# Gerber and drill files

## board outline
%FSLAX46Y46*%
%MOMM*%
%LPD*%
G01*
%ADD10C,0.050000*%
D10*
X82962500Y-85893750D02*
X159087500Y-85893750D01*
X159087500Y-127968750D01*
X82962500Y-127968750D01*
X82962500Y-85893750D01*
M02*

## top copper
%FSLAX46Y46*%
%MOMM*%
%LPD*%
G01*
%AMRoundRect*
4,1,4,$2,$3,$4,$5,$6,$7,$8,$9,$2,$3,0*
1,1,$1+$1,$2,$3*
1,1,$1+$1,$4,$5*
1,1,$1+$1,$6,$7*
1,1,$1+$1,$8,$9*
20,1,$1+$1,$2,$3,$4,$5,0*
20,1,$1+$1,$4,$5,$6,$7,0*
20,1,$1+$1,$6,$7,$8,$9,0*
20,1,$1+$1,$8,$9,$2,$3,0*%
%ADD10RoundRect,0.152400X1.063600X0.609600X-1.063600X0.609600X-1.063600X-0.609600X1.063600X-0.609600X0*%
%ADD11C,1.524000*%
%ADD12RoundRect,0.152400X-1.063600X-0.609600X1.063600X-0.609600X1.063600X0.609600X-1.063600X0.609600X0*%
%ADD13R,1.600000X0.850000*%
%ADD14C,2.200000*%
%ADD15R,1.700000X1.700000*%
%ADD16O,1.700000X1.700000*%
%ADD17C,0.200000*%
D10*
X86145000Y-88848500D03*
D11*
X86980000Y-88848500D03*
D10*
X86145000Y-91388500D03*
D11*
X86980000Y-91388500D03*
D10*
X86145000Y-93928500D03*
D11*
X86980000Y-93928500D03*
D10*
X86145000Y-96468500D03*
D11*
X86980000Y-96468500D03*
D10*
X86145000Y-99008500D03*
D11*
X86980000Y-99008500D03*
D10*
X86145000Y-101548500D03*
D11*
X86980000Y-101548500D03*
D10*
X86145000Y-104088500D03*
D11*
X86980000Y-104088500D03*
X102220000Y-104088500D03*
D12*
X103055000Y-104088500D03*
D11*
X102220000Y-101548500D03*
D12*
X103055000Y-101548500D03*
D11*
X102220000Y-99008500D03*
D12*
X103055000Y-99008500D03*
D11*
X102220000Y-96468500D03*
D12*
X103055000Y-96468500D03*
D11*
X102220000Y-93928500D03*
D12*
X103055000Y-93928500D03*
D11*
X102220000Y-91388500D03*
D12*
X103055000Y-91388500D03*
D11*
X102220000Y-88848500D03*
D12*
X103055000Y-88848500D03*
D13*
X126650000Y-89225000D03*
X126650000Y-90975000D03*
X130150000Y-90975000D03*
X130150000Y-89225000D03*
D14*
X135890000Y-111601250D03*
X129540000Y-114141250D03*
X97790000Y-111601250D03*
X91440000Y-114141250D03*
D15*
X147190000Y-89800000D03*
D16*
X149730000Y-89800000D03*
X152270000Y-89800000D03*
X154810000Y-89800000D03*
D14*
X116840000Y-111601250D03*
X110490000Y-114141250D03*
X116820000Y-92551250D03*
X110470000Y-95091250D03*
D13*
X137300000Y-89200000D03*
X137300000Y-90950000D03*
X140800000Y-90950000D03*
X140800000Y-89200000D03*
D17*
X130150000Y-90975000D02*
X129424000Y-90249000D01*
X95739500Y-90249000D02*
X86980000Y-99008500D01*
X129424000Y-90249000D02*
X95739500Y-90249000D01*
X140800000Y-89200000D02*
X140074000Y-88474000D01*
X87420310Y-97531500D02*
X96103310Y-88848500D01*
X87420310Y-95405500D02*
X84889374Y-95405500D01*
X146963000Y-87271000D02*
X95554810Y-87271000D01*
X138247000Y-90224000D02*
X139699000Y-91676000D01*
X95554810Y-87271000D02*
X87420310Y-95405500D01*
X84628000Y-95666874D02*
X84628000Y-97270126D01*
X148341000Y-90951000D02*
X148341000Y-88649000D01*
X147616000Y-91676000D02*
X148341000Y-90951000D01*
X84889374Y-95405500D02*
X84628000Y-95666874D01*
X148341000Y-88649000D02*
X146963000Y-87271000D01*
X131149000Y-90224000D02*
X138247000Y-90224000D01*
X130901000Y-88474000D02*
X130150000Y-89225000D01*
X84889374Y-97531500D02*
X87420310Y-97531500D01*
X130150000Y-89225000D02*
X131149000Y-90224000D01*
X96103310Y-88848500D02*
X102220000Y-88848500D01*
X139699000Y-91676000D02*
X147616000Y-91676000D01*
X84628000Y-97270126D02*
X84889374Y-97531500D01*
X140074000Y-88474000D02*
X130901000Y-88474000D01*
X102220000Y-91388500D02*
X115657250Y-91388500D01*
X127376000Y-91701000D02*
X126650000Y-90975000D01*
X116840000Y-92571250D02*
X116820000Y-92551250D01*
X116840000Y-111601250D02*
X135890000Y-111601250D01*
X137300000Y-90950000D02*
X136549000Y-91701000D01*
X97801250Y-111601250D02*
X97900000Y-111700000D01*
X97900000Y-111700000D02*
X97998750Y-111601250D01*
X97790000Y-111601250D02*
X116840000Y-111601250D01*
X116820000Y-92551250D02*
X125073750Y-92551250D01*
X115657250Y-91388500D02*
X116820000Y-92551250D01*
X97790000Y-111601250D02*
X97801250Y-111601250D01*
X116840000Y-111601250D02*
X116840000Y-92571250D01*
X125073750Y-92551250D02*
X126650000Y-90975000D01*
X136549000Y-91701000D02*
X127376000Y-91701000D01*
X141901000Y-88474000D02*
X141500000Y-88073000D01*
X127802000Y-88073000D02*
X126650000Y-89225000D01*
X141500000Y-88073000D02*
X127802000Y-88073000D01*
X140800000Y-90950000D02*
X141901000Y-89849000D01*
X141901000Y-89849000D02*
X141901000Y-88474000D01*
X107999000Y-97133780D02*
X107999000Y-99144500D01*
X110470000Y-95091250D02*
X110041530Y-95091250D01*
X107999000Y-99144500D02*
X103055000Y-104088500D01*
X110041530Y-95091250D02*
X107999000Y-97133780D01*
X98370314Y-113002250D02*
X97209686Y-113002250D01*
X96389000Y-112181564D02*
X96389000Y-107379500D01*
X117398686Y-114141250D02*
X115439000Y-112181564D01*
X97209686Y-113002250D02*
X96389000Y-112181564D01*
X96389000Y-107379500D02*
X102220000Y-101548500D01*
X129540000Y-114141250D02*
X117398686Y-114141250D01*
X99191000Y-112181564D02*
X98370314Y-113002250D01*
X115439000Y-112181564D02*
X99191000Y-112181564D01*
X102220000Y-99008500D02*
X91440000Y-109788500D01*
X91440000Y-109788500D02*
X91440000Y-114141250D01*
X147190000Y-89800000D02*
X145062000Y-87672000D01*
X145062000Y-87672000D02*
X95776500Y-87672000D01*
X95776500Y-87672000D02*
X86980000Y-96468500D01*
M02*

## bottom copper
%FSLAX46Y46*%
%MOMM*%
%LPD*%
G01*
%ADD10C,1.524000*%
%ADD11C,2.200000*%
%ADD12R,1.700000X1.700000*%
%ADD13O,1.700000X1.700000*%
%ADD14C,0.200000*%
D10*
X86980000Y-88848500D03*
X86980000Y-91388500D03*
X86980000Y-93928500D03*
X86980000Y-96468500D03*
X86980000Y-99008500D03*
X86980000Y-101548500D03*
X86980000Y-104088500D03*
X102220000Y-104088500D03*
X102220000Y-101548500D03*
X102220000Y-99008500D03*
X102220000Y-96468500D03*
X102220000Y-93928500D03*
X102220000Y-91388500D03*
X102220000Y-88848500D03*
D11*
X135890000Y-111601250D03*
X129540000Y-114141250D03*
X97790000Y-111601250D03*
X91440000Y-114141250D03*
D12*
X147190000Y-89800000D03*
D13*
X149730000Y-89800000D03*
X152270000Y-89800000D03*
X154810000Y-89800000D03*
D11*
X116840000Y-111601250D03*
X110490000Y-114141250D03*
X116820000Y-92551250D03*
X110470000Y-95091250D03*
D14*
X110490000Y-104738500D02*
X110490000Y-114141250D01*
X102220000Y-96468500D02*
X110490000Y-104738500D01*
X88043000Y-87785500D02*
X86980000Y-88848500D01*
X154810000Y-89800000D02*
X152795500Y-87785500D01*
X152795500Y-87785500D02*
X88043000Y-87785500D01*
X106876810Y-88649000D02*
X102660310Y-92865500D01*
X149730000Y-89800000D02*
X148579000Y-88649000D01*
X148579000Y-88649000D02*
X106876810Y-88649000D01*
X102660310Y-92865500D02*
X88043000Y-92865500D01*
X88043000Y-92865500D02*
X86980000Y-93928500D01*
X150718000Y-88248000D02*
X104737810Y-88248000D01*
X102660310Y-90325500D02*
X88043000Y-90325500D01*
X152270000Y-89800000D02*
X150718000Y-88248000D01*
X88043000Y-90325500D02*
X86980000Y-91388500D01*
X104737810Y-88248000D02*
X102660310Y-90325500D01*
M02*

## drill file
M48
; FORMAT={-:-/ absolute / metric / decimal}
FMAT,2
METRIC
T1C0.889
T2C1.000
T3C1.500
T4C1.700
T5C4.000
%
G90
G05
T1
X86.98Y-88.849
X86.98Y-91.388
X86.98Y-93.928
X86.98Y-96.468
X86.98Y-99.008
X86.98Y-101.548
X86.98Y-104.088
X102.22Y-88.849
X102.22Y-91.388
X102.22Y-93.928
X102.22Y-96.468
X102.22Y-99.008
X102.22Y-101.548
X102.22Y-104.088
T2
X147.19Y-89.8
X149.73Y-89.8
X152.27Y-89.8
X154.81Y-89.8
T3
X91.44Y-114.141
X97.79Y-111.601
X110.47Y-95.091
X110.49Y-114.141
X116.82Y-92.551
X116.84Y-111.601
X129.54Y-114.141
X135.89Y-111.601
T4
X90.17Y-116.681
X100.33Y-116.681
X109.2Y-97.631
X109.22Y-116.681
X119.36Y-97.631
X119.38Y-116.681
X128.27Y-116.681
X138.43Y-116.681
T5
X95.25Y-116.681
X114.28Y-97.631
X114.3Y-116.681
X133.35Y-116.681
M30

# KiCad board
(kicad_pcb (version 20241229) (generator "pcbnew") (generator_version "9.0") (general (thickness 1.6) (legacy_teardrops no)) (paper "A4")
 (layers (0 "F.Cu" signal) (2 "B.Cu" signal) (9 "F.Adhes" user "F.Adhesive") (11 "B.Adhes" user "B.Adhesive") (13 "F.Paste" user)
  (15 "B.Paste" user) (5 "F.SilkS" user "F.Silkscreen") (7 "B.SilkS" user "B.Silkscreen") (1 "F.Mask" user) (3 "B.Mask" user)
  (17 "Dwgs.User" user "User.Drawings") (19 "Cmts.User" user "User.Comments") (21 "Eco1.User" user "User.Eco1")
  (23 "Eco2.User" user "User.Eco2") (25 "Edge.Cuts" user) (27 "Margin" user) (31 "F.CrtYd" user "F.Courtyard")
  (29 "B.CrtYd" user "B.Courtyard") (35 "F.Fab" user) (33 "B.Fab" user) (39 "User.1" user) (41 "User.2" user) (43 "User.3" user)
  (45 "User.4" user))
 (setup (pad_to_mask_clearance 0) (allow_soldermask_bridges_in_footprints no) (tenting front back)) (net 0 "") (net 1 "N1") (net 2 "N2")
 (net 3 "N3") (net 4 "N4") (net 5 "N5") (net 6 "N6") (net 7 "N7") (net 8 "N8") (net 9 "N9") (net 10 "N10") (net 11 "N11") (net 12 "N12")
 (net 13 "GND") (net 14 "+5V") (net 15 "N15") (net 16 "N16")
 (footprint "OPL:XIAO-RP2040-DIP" (layer "F.Cu") (at 94.6 96.4685)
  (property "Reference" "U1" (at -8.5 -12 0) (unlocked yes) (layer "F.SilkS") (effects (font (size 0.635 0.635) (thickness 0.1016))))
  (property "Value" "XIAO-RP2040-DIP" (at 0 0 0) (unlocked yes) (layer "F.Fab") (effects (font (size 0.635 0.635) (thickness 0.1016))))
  (pad "1" smd roundrect (at -8.455 -7.62 180) (size 2.432 1.524) (layers "F.Cu" "F.Mask") (roundrect_rratio 0.1) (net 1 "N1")
   (thermal_bridge_angle 45))
  (pad "1" thru_hole circle (at -7.62 -7.62 180) (size 1.524 1.524) (drill 0.889) (layers "*.Cu" "*.Mask") (remove_unused_layers no)
   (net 1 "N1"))
  (pad "2" smd roundrect (at -8.455 -5.08 180) (size 2.432 1.524) (layers "F.Cu" "F.Mask") (roundrect_rratio 0.1) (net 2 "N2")
   (thermal_bridge_angle 45))
  (pad "2" thru_hole circle (at -7.62 -5.08 180) (size 1.524 1.524) (drill 0.889) (layers "*.Cu" "*.Mask") (remove_unused_layers no)
   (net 2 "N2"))
  (pad "3" smd roundrect (at -8.455 -2.54 180) (size 2.432 1.524) (layers "F.Cu" "F.Mask") (roundrect_rratio 0.1) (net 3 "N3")
   (thermal_bridge_angle 45))
  (pad "3" thru_hole circle (at -7.62 -2.54 180) (size 1.524 1.524) (drill 0.889) (layers "*.Cu" "*.Mask") (remove_unused_layers no)
   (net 3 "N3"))
  (pad "4" smd roundrect (at -8.455 0 180) (size 2.432 1.524) (layers "F.Cu" "F.Mask") (roundrect_rratio 0.1) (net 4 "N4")
   (thermal_bridge_angle 45))
  (pad "4" thru_hole circle (at -7.62 0 180) (size 1.524 1.524) (drill 0.889) (layers "*.Cu" "*.Mask") (remove_unused_layers no)
   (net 4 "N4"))
  (pad "5" smd roundrect (at -8.455 2.54 180) (size 2.432 1.524) (layers "F.Cu" "F.Mask") (roundrect_rratio 0.1) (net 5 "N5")
   (thermal_bridge_angle 45))
  (pad "5" thru_hole circle (at -7.62 2.54 180) (size 1.524 1.524) (drill 0.889) (layers "*.Cu" "*.Mask") (remove_unused_layers no)
   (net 5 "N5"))
  (pad "6" smd roundrect (at -8.455 5.08 180) (size 2.432 1.524) (layers "F.Cu" "F.Mask") (roundrect_rratio 0.1) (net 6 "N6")
   (thermal_bridge_angle 45))
  (pad "6" thru_hole circle (at -7.62 5.08 180) (size 1.524 1.524) (drill 0.889) (layers "*.Cu" "*.Mask") (remove_unused_layers no)
   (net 6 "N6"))
  (pad "7" smd roundrect (at -8.455 7.62 180) (size 2.432 1.524) (layers "F.Cu" "F.Mask") (roundrect_rratio 0.1) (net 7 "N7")
   (thermal_bridge_angle 45))
  (pad "7" thru_hole circle (at -7.62 7.62 180) (size 1.524 1.524) (drill 0.889) (layers "*.Cu" "*.Mask") (remove_unused_layers no)
   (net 7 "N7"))
  (pad "8" thru_hole circle (at 7.62 7.62) (size 1.524 1.524) (drill 0.889) (layers "*.Cu" "*.Mask") (remove_unused_layers no) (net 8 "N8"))
  (pad "8" smd roundrect (at 8.455 7.62) (size 2.432 1.524) (layers "F.Cu" "F.Mask") (roundrect_rratio 0.1) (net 8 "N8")
   (thermal_bridge_angle 45))
  (pad "9" thru_hole circle (at 7.62 5.08) (size 1.524 1.524) (drill 0.889) (layers "*.Cu" "*.Mask") (remove_unused_layers no) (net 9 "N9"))
  (pad "9" smd roundrect (at 8.455 5.08) (size 2.432 1.524) (layers "F.Cu" "F.Mask") (roundrect_rratio 0.1) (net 9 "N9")
   (thermal_bridge_angle 45))
  (pad "10" thru_hole circle (at 7.62 2.54) (size 1.524 1.524) (drill 0.889) (layers "*.Cu" "*.Mask") (remove_unused_layers no)
   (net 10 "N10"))
  (pad "10" smd roundrect (at 8.455 2.54) (size 2.432 1.524) (layers "F.Cu" "F.Mask") (roundrect_rratio 0.1) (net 10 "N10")
   (thermal_bridge_angle 45))
  (pad "11" thru_hole circle (at 7.62 0) (size 1.524 1.524) (drill 0.889) (layers "*.Cu" "*.Mask") (remove_unused_layers no) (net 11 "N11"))
  (pad "11" smd roundrect (at 8.455 0) (size 2.432 1.524) (layers "F.Cu" "F.Mask") (roundrect_rratio 0.1) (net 11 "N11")
   (thermal_bridge_angle 45))
  (pad "12" thru_hole circle (at 7.62 -2.54) (size 1.524 1.524) (drill 0.889) (layers "*.Cu" "*.Mask") (remove_unused_layers no)
   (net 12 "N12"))
  (pad "12" smd roundrect (at 8.455 -2.54) (size 2.432 1.524) (layers "F.Cu" "F.Mask") (roundrect_rratio 0.1) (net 12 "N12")
   (thermal_bridge_angle 45))
  (pad "13" thru_hole circle (at 7.62 -5.08) (size 1.524 1.524) (drill 0.889) (layers "*.Cu" "*.Mask") (remove_unused_layers no)
   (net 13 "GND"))
  (pad "13" smd roundrect (at 8.455 -5.08) (size 2.432 1.524) (layers "F.Cu" "F.Mask") (roundrect_rratio 0.1) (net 13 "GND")
   (thermal_bridge_angle 45))
  (pad "14" thru_hole circle (at 7.62 -7.62) (size 1.524 1.524) (drill 0.889) (layers "*.Cu" "*.Mask") (remove_unused_layers no)
   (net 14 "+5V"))
  (pad "14" smd roundrect (at 8.455 -7.62) (size 2.432 1.524) (layers "F.Cu" "F.Mask") (roundrect_rratio 0.1) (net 14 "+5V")
   (thermal_bridge_angle 45)))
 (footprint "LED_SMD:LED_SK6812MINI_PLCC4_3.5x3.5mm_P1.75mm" (layer "F.Cu") (at 128.4 90.1)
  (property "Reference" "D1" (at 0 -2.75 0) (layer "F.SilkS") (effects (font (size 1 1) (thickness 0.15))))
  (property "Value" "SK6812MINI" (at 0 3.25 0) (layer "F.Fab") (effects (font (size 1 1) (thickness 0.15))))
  (pad "1" smd rect (at -1.75 -0.875) (size 1.6 0.85) (layers "F.Cu" "F.Mask" "F.Paste") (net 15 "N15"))
  (pad "2" smd rect (at -1.75 0.875) (size 1.6 0.85) (layers "F.Cu" "F.Mask" "F.Paste") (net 13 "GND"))
  (pad "3" smd rect (at 1.75 0.875) (size 1.6 0.85) (layers "F.Cu" "F.Mask" "F.Paste") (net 5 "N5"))
  (pad "4" smd rect (at 1.75 -0.875) (size 1.6 0.85) (layers "F.Cu" "F.Mask" "F.Paste") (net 14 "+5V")))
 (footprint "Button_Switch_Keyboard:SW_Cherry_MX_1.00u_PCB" (layer "F.Cu") (at 135.89 111.60125)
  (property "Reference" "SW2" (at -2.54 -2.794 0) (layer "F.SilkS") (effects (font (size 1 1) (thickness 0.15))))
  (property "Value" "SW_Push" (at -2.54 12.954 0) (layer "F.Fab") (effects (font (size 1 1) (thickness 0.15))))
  (pad "" np_thru_hole circle (at -7.62 5.08) (size 1.7 1.7) (drill 1.7) (layers "*.Cu" "*.Mask"))
  (pad "" np_thru_hole circle (at -2.54 5.08) (size 4 4) (drill 4) (layers "*.Cu" "*.Mask"))
  (pad "" np_thru_hole circle (at 2.54 5.08) (size 1.7 1.7) (drill 1.7) (layers "*.Cu" "*.Mask"))
  (pad "1" thru_hole circle (at 0 0) (size 2.2 2.2) (drill 1.5) (layers "*.Cu" "*.Mask") (remove_unused_layers no) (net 13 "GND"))
  (pad "2" thru_hole circle (at -6.35 2.54) (size 2.2 2.2) (drill 1.5) (layers "*.Cu" "*.Mask") (remove_unused_layers no) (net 9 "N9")))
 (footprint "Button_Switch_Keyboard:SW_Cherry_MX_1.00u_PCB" (layer "F.Cu") (at 97.79 111.60125)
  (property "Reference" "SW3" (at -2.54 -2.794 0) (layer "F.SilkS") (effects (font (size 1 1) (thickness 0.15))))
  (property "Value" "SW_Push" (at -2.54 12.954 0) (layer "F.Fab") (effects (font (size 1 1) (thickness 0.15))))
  (pad "" np_thru_hole circle (at -7.62 5.08) (size 1.7 1.7) (drill 1.7) (layers "*.Cu" "*.Mask"))
  (pad "" np_thru_hole circle (at -2.54 5.08) (size 4 4) (drill 4) (layers "*.Cu" "*.Mask"))
  (pad "" np_thru_hole circle (at 2.54 5.08) (size 1.7 1.7) (drill 1.7) (layers "*.Cu" "*.Mask"))
  (pad "1" thru_hole circle (at 0 0) (size 2.2 2.2) (drill 1.5) (layers "*.Cu" "*.Mask") (remove_unused_layers no) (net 13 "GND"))
  (pad "2" thru_hole circle (at -6.35 2.54) (size 2.2 2.2) (drill 1.5) (layers "*.Cu" "*.Mask") (remove_unused_layers no) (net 10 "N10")))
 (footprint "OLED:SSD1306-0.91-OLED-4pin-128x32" (layer "F.Cu") (at 145 126.3 90)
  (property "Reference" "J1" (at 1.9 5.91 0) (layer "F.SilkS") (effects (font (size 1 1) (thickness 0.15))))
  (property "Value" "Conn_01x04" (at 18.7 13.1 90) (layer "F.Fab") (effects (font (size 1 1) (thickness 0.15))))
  (pad "1" thru_hole rect (at 36.5 2.19 90) (size 1.7 1.7) (drill 1) (layers "*.Cu" "*.Mask") (remove_unused_layers no) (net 4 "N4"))
  (pad "2" thru_hole oval (at 36.5 4.73 90) (size 1.7 1.7) (drill 1) (layers "*.Cu" "*.Mask") (remove_unused_layers no) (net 3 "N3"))
  (pad "3" thru_hole oval (at 36.5 7.27 90) (size 1.7 1.7) (drill 1) (layers "*.Cu" "*.Mask") (remove_unused_layers no) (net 2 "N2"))
  (pad "4" thru_hole oval (at 36.5 9.81 90) (size 1.7 1.7) (drill 1) (layers "*.Cu" "*.Mask") (remove_unused_layers no) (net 1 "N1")))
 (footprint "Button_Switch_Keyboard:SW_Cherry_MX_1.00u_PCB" (layer "F.Cu") (at 116.84 111.60125)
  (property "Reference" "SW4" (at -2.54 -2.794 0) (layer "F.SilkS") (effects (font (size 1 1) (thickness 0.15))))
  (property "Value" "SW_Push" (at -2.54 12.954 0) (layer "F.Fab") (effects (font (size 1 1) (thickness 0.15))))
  (pad "" np_thru_hole circle (at -7.62 5.08) (size 1.7 1.7) (drill 1.7) (layers "*.Cu" "*.Mask"))
  (pad "" np_thru_hole circle (at -2.54 5.08) (size 4 4) (drill 4) (layers "*.Cu" "*.Mask"))
  (pad "" np_thru_hole circle (at 2.54 5.08) (size 1.7 1.7) (drill 1.7) (layers "*.Cu" "*.Mask"))
  (pad "1" thru_hole circle (at 0 0) (size 2.2 2.2) (drill 1.5) (layers "*.Cu" "*.Mask") (remove_unused_layers no) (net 13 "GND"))
  (pad "2" thru_hole circle (at -6.35 2.54) (size 2.2 2.2) (drill 1.5) (layers "*.Cu" "*.Mask") (remove_unused_layers no) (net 11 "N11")))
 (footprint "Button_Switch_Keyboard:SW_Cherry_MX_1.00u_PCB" (layer "F.Cu") (at 116.82 92.55125)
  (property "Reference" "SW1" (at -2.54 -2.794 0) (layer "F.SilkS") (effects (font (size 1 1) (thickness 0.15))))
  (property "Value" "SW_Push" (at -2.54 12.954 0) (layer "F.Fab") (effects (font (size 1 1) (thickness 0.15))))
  (pad "" np_thru_hole circle (at -7.62 5.08) (size 1.7 1.7) (drill 1.7) (layers "*.Cu" "*.Mask"))
  (pad "" np_thru_hole circle (at -2.54 5.08) (size 4 4) (drill 4) (layers "*.Cu" "*.Mask"))
  (pad "" np_thru_hole circle (at 2.54 5.08) (size 1.7 1.7) (drill 1.7) (layers "*.Cu" "*.Mask"))
  (pad "1" thru_hole circle (at 0 0) (size 2.2 2.2) (drill 1.5) (layers "*.Cu" "*.Mask") (remove_unused_layers no) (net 13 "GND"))
  (pad "2" thru_hole circle (at -6.35 2.54) (size 2.2 2.2) (drill 1.5) (layers "*.Cu" "*.Mask") (remove_unused_layers no) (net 8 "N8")))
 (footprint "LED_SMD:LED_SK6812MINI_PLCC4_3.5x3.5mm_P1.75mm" (layer "F.Cu") (at 139.05 90.075)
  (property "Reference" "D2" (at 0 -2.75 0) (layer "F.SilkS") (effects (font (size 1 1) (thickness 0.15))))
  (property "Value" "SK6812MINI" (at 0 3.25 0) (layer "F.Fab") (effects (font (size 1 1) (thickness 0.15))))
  (pad "1" smd rect (at -1.75 -0.875) (size 1.6 0.85) (layers "F.Cu" "F.Mask" "F.Paste") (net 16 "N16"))
  (pad "2" smd rect (at -1.75 0.875) (size 1.6 0.85) (layers "F.Cu" "F.Mask" "F.Paste") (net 13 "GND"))
  (pad "3" smd rect (at 1.75 0.875) (size 1.6 0.85) (layers "F.Cu" "F.Mask" "F.Paste") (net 15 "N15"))
  (pad "4" smd rect (at 1.75 -0.875) (size 1.6 0.85) (layers "F.Cu" "F.Mask" "F.Paste") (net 14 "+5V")))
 (gr_rect (start 82.9625 85.89375) (end 159.0875 127.96875) (stroke (width 0.05) (type default)) (fill no) (layer "Edge.Cuts"))
 (segment (start 130.15 90.975) (end 129.424 90.249) (width 0.2) (layer "F.Cu") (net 5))
 (segment (start 95.7395 90.249) (end 86.98 99.0085) (width 0.2) (layer "F.Cu") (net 5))
 (segment (start 129.424 90.249) (end 95.7395 90.249) (width 0.2) (layer "F.Cu") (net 5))
 (segment (start 140.8 89.2) (end 140.074 88.474) (width 0.2) (layer "F.Cu") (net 14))
 (segment (start 87.42031 97.5315) (end 96.10331 88.8485) (width 0.2) (layer "F.Cu") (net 14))
 (segment (start 87.42031 95.4055) (end 84.889374 95.4055) (width 0.2) (layer "F.Cu") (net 14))
 (segment (start 146.963 87.271) (end 95.55481 87.271) (width 0.2) (layer "F.Cu") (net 14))
 (segment (start 138.247 90.224) (end 139.699 91.676) (width 0.2) (layer "F.Cu") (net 14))
 (segment (start 95.55481 87.271) (end 87.42031 95.4055) (width 0.2) (layer "F.Cu") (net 14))
 (segment (start 84.628 95.666874) (end 84.628 97.270126) (width 0.2) (layer "F.Cu") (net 14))
 (segment (start 148.341 90.951) (end 148.341 88.649) (width 0.2) (layer "F.Cu") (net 14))
 (segment (start 147.616 91.676) (end 148.341 90.951) (width 0.2) (layer "F.Cu") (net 14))
 (segment (start 84.889374 95.4055) (end 84.628 95.666874) (width 0.2) (layer "F.Cu") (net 14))
 (segment (start 148.341 88.649) (end 146.963 87.271) (width 0.2) (layer "F.Cu") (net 14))
 (segment (start 131.149 90.224) (end 138.247 90.224) (width 0.2) (layer "F.Cu") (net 14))
 (segment (start 130.901 88.474) (end 130.15 89.225) (width 0.2) (layer "F.Cu") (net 14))
 (segment (start 84.889374 97.5315) (end 87.42031 97.5315) (width 0.2) (layer "F.Cu") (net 14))
 (segment (start 130.15 89.225) (end 131.149 90.224) (width 0.2) (layer "F.Cu") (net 14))
 (segment (start 96.10331 88.8485) (end 102.22 88.8485) (width 0.2) (layer "F.Cu") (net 14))
 (segment (start 139.699 91.676) (end 147.616 91.676) (width 0.2) (layer "F.Cu") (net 14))
 (segment (start 84.628 97.270126) (end 84.889374 97.5315) (width 0.2) (layer "F.Cu") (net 14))
 (segment (start 140.074 88.474) (end 130.901 88.474) (width 0.2) (layer "F.Cu") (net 14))
 (segment (start 102.22 91.3885) (end 115.65725 91.3885) (width 0.2) (layer "F.Cu") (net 13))
 (segment (start 127.376 91.701) (end 126.65 90.975) (width 0.2) (layer "F.Cu") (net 13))
 (segment (start 116.84 92.57125) (end 116.82 92.55125) (width 0.2) (layer "F.Cu") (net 13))
 (segment (start 116.84 111.60125) (end 135.89 111.60125) (width 0.2) (layer "F.Cu") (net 13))
 (segment (start 137.3 90.95) (end 136.549 91.701) (width 0.2) (layer "F.Cu") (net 13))
 (segment (start 97.80125 111.60125) (end 97.9 111.7) (width 0.2) (layer "F.Cu") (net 13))
 (segment (start 97.9 111.7) (end 97.99875 111.60125) (width 0.2) (layer "F.Cu") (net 13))
 (segment (start 97.79 111.60125) (end 116.84 111.60125) (width 0.2) (layer "F.Cu") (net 13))
 (segment (start 116.82 92.55125) (end 125.07375 92.55125) (width 0.2) (layer "F.Cu") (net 13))
 (segment (start 115.65725 91.3885) (end 116.82 92.55125) (width 0.2) (layer "F.Cu") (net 13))
 (segment (start 97.79 111.60125) (end 97.80125 111.60125) (width 0.2) (layer "F.Cu") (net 13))
 (segment (start 116.84 111.60125) (end 116.84 92.57125) (width 0.2) (layer "F.Cu") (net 13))
 (segment (start 125.07375 92.55125) (end 126.65 90.975) (width 0.2) (layer "F.Cu") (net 13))
 (segment (start 136.549 91.701) (end 127.376 91.701) (width 0.2) (layer "F.Cu") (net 13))
 (segment (start 141.901 88.474) (end 141.5 88.073) (width 0.2) (layer "F.Cu") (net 15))
 (segment (start 127.802 88.073) (end 126.65 89.225) (width 0.2) (layer "F.Cu") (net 15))
 (segment (start 141.5 88.073) (end 127.802 88.073) (width 0.2) (layer "F.Cu") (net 15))
 (segment (start 140.8 90.95) (end 141.901 89.849) (width 0.2) (layer "F.Cu") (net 15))
 (segment (start 141.901 89.849) (end 141.901 88.474) (width 0.2) (layer "F.Cu") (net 15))
 (segment (start 107.999 97.13378) (end 107.999 99.1445) (width 0.2) (layer "F.Cu") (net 8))
 (segment (start 110.47 95.09125) (end 110.04153 95.09125) (width 0.2) (layer "F.Cu") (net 8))
 (segment (start 107.999 99.1445) (end 103.055 104.0885) (width 0.2) (layer "F.Cu") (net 8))
 (segment (start 110.04153 95.09125) (end 107.999 97.13378) (width 0.2) (layer "F.Cu") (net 8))
 (segment (start 98.370314 113.00225) (end 97.209686 113.00225) (width 0.2) (layer "F.Cu") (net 9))
 (segment (start 96.389 112.181564) (end 96.389 107.3795) (width 0.2) (layer "F.Cu") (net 9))
 (segment (start 117.398686 114.14125) (end 115.439 112.181564) (width 0.2) (layer "F.Cu") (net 9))
 (segment (start 97.209686 113.00225) (end 96.389 112.181564) (width 0.2) (layer "F.Cu") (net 9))
 (segment (start 96.389 107.3795) (end 102.22 101.5485) (width 0.2) (layer "F.Cu") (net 9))
 (segment (start 129.54 114.14125) (end 117.398686 114.14125) (width 0.2) (layer "F.Cu") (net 9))
 (segment (start 99.191 112.181564) (end 98.370314 113.00225) (width 0.2) (layer "F.Cu") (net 9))
 (segment (start 115.439 112.181564) (end 99.191 112.181564) (width 0.2) (layer "F.Cu") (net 9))
 (segment (start 102.22 99.0085) (end 91.44 109.7885) (width 0.2) (layer "F.Cu") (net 10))
 (segment (start 91.44 109.7885) (end 91.44 114.14125) (width 0.2) (layer "F.Cu") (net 10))
 (segment (start 110.49 104.7385) (end 110.49 114.14125) (width 0.2) (layer "B.Cu") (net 11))
 (segment (start 102.22 96.4685) (end 110.49 104.7385) (width 0.2) (layer "B.Cu") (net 11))
 (segment (start 88.043 87.7855) (end 86.98 88.8485) (width 0.2) (layer "B.Cu") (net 1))
 (segment (start 154.81 89.8) (end 152.7955 87.7855) (width 0.2) (layer "B.Cu") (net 1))
 (segment (start 152.7955 87.7855) (end 88.043 87.7855) (width 0.2) (layer "B.Cu") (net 1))
 (segment (start 106.87681 88.649) (end 102.66031 92.8655) (width 0.2) (layer "B.Cu") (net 3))
 (segment (start 149.73 89.8) (end 148.579 88.649) (width 0.2) (layer "B.Cu") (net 3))
 (segment (start 148.579 88.649) (end 106.87681 88.649) (width 0.2) (layer "B.Cu") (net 3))
 (segment (start 102.66031 92.8655) (end 88.043 92.8655) (width 0.2) (layer "B.Cu") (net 3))
 (segment (start 88.043 92.8655) (end 86.98 93.9285) (width 0.2) (layer "B.Cu") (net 3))
 (segment (start 150.718 88.248) (end 104.73781 88.248) (width 0.2) (layer "B.Cu") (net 2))
 (segment (start 102.66031 90.3255) (end 88.043 90.3255) (width 0.2) (layer "B.Cu") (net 2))
 (segment (start 152.27 89.8) (end 150.718 88.248) (width 0.2) (layer "B.Cu") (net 2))
 (segment (start 88.043 90.3255) (end 86.98 91.3885) (width 0.2) (layer "B.Cu") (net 2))
 (segment (start 104.73781 88.248) (end 102.66031 90.3255) (width 0.2) (layer "B.Cu") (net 2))
 (segment (start 147.19 89.8) (end 145.062 87.672) (width 0.2) (layer "F.Cu") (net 4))
 (segment (start 145.062 87.672) (end 95.7765 87.672) (width 0.2) (layer "F.Cu") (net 4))
 (segment (start 95.7765 87.672) (end 86.98 96.4685) (width 0.2) (layer "F.Cu") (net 4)))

